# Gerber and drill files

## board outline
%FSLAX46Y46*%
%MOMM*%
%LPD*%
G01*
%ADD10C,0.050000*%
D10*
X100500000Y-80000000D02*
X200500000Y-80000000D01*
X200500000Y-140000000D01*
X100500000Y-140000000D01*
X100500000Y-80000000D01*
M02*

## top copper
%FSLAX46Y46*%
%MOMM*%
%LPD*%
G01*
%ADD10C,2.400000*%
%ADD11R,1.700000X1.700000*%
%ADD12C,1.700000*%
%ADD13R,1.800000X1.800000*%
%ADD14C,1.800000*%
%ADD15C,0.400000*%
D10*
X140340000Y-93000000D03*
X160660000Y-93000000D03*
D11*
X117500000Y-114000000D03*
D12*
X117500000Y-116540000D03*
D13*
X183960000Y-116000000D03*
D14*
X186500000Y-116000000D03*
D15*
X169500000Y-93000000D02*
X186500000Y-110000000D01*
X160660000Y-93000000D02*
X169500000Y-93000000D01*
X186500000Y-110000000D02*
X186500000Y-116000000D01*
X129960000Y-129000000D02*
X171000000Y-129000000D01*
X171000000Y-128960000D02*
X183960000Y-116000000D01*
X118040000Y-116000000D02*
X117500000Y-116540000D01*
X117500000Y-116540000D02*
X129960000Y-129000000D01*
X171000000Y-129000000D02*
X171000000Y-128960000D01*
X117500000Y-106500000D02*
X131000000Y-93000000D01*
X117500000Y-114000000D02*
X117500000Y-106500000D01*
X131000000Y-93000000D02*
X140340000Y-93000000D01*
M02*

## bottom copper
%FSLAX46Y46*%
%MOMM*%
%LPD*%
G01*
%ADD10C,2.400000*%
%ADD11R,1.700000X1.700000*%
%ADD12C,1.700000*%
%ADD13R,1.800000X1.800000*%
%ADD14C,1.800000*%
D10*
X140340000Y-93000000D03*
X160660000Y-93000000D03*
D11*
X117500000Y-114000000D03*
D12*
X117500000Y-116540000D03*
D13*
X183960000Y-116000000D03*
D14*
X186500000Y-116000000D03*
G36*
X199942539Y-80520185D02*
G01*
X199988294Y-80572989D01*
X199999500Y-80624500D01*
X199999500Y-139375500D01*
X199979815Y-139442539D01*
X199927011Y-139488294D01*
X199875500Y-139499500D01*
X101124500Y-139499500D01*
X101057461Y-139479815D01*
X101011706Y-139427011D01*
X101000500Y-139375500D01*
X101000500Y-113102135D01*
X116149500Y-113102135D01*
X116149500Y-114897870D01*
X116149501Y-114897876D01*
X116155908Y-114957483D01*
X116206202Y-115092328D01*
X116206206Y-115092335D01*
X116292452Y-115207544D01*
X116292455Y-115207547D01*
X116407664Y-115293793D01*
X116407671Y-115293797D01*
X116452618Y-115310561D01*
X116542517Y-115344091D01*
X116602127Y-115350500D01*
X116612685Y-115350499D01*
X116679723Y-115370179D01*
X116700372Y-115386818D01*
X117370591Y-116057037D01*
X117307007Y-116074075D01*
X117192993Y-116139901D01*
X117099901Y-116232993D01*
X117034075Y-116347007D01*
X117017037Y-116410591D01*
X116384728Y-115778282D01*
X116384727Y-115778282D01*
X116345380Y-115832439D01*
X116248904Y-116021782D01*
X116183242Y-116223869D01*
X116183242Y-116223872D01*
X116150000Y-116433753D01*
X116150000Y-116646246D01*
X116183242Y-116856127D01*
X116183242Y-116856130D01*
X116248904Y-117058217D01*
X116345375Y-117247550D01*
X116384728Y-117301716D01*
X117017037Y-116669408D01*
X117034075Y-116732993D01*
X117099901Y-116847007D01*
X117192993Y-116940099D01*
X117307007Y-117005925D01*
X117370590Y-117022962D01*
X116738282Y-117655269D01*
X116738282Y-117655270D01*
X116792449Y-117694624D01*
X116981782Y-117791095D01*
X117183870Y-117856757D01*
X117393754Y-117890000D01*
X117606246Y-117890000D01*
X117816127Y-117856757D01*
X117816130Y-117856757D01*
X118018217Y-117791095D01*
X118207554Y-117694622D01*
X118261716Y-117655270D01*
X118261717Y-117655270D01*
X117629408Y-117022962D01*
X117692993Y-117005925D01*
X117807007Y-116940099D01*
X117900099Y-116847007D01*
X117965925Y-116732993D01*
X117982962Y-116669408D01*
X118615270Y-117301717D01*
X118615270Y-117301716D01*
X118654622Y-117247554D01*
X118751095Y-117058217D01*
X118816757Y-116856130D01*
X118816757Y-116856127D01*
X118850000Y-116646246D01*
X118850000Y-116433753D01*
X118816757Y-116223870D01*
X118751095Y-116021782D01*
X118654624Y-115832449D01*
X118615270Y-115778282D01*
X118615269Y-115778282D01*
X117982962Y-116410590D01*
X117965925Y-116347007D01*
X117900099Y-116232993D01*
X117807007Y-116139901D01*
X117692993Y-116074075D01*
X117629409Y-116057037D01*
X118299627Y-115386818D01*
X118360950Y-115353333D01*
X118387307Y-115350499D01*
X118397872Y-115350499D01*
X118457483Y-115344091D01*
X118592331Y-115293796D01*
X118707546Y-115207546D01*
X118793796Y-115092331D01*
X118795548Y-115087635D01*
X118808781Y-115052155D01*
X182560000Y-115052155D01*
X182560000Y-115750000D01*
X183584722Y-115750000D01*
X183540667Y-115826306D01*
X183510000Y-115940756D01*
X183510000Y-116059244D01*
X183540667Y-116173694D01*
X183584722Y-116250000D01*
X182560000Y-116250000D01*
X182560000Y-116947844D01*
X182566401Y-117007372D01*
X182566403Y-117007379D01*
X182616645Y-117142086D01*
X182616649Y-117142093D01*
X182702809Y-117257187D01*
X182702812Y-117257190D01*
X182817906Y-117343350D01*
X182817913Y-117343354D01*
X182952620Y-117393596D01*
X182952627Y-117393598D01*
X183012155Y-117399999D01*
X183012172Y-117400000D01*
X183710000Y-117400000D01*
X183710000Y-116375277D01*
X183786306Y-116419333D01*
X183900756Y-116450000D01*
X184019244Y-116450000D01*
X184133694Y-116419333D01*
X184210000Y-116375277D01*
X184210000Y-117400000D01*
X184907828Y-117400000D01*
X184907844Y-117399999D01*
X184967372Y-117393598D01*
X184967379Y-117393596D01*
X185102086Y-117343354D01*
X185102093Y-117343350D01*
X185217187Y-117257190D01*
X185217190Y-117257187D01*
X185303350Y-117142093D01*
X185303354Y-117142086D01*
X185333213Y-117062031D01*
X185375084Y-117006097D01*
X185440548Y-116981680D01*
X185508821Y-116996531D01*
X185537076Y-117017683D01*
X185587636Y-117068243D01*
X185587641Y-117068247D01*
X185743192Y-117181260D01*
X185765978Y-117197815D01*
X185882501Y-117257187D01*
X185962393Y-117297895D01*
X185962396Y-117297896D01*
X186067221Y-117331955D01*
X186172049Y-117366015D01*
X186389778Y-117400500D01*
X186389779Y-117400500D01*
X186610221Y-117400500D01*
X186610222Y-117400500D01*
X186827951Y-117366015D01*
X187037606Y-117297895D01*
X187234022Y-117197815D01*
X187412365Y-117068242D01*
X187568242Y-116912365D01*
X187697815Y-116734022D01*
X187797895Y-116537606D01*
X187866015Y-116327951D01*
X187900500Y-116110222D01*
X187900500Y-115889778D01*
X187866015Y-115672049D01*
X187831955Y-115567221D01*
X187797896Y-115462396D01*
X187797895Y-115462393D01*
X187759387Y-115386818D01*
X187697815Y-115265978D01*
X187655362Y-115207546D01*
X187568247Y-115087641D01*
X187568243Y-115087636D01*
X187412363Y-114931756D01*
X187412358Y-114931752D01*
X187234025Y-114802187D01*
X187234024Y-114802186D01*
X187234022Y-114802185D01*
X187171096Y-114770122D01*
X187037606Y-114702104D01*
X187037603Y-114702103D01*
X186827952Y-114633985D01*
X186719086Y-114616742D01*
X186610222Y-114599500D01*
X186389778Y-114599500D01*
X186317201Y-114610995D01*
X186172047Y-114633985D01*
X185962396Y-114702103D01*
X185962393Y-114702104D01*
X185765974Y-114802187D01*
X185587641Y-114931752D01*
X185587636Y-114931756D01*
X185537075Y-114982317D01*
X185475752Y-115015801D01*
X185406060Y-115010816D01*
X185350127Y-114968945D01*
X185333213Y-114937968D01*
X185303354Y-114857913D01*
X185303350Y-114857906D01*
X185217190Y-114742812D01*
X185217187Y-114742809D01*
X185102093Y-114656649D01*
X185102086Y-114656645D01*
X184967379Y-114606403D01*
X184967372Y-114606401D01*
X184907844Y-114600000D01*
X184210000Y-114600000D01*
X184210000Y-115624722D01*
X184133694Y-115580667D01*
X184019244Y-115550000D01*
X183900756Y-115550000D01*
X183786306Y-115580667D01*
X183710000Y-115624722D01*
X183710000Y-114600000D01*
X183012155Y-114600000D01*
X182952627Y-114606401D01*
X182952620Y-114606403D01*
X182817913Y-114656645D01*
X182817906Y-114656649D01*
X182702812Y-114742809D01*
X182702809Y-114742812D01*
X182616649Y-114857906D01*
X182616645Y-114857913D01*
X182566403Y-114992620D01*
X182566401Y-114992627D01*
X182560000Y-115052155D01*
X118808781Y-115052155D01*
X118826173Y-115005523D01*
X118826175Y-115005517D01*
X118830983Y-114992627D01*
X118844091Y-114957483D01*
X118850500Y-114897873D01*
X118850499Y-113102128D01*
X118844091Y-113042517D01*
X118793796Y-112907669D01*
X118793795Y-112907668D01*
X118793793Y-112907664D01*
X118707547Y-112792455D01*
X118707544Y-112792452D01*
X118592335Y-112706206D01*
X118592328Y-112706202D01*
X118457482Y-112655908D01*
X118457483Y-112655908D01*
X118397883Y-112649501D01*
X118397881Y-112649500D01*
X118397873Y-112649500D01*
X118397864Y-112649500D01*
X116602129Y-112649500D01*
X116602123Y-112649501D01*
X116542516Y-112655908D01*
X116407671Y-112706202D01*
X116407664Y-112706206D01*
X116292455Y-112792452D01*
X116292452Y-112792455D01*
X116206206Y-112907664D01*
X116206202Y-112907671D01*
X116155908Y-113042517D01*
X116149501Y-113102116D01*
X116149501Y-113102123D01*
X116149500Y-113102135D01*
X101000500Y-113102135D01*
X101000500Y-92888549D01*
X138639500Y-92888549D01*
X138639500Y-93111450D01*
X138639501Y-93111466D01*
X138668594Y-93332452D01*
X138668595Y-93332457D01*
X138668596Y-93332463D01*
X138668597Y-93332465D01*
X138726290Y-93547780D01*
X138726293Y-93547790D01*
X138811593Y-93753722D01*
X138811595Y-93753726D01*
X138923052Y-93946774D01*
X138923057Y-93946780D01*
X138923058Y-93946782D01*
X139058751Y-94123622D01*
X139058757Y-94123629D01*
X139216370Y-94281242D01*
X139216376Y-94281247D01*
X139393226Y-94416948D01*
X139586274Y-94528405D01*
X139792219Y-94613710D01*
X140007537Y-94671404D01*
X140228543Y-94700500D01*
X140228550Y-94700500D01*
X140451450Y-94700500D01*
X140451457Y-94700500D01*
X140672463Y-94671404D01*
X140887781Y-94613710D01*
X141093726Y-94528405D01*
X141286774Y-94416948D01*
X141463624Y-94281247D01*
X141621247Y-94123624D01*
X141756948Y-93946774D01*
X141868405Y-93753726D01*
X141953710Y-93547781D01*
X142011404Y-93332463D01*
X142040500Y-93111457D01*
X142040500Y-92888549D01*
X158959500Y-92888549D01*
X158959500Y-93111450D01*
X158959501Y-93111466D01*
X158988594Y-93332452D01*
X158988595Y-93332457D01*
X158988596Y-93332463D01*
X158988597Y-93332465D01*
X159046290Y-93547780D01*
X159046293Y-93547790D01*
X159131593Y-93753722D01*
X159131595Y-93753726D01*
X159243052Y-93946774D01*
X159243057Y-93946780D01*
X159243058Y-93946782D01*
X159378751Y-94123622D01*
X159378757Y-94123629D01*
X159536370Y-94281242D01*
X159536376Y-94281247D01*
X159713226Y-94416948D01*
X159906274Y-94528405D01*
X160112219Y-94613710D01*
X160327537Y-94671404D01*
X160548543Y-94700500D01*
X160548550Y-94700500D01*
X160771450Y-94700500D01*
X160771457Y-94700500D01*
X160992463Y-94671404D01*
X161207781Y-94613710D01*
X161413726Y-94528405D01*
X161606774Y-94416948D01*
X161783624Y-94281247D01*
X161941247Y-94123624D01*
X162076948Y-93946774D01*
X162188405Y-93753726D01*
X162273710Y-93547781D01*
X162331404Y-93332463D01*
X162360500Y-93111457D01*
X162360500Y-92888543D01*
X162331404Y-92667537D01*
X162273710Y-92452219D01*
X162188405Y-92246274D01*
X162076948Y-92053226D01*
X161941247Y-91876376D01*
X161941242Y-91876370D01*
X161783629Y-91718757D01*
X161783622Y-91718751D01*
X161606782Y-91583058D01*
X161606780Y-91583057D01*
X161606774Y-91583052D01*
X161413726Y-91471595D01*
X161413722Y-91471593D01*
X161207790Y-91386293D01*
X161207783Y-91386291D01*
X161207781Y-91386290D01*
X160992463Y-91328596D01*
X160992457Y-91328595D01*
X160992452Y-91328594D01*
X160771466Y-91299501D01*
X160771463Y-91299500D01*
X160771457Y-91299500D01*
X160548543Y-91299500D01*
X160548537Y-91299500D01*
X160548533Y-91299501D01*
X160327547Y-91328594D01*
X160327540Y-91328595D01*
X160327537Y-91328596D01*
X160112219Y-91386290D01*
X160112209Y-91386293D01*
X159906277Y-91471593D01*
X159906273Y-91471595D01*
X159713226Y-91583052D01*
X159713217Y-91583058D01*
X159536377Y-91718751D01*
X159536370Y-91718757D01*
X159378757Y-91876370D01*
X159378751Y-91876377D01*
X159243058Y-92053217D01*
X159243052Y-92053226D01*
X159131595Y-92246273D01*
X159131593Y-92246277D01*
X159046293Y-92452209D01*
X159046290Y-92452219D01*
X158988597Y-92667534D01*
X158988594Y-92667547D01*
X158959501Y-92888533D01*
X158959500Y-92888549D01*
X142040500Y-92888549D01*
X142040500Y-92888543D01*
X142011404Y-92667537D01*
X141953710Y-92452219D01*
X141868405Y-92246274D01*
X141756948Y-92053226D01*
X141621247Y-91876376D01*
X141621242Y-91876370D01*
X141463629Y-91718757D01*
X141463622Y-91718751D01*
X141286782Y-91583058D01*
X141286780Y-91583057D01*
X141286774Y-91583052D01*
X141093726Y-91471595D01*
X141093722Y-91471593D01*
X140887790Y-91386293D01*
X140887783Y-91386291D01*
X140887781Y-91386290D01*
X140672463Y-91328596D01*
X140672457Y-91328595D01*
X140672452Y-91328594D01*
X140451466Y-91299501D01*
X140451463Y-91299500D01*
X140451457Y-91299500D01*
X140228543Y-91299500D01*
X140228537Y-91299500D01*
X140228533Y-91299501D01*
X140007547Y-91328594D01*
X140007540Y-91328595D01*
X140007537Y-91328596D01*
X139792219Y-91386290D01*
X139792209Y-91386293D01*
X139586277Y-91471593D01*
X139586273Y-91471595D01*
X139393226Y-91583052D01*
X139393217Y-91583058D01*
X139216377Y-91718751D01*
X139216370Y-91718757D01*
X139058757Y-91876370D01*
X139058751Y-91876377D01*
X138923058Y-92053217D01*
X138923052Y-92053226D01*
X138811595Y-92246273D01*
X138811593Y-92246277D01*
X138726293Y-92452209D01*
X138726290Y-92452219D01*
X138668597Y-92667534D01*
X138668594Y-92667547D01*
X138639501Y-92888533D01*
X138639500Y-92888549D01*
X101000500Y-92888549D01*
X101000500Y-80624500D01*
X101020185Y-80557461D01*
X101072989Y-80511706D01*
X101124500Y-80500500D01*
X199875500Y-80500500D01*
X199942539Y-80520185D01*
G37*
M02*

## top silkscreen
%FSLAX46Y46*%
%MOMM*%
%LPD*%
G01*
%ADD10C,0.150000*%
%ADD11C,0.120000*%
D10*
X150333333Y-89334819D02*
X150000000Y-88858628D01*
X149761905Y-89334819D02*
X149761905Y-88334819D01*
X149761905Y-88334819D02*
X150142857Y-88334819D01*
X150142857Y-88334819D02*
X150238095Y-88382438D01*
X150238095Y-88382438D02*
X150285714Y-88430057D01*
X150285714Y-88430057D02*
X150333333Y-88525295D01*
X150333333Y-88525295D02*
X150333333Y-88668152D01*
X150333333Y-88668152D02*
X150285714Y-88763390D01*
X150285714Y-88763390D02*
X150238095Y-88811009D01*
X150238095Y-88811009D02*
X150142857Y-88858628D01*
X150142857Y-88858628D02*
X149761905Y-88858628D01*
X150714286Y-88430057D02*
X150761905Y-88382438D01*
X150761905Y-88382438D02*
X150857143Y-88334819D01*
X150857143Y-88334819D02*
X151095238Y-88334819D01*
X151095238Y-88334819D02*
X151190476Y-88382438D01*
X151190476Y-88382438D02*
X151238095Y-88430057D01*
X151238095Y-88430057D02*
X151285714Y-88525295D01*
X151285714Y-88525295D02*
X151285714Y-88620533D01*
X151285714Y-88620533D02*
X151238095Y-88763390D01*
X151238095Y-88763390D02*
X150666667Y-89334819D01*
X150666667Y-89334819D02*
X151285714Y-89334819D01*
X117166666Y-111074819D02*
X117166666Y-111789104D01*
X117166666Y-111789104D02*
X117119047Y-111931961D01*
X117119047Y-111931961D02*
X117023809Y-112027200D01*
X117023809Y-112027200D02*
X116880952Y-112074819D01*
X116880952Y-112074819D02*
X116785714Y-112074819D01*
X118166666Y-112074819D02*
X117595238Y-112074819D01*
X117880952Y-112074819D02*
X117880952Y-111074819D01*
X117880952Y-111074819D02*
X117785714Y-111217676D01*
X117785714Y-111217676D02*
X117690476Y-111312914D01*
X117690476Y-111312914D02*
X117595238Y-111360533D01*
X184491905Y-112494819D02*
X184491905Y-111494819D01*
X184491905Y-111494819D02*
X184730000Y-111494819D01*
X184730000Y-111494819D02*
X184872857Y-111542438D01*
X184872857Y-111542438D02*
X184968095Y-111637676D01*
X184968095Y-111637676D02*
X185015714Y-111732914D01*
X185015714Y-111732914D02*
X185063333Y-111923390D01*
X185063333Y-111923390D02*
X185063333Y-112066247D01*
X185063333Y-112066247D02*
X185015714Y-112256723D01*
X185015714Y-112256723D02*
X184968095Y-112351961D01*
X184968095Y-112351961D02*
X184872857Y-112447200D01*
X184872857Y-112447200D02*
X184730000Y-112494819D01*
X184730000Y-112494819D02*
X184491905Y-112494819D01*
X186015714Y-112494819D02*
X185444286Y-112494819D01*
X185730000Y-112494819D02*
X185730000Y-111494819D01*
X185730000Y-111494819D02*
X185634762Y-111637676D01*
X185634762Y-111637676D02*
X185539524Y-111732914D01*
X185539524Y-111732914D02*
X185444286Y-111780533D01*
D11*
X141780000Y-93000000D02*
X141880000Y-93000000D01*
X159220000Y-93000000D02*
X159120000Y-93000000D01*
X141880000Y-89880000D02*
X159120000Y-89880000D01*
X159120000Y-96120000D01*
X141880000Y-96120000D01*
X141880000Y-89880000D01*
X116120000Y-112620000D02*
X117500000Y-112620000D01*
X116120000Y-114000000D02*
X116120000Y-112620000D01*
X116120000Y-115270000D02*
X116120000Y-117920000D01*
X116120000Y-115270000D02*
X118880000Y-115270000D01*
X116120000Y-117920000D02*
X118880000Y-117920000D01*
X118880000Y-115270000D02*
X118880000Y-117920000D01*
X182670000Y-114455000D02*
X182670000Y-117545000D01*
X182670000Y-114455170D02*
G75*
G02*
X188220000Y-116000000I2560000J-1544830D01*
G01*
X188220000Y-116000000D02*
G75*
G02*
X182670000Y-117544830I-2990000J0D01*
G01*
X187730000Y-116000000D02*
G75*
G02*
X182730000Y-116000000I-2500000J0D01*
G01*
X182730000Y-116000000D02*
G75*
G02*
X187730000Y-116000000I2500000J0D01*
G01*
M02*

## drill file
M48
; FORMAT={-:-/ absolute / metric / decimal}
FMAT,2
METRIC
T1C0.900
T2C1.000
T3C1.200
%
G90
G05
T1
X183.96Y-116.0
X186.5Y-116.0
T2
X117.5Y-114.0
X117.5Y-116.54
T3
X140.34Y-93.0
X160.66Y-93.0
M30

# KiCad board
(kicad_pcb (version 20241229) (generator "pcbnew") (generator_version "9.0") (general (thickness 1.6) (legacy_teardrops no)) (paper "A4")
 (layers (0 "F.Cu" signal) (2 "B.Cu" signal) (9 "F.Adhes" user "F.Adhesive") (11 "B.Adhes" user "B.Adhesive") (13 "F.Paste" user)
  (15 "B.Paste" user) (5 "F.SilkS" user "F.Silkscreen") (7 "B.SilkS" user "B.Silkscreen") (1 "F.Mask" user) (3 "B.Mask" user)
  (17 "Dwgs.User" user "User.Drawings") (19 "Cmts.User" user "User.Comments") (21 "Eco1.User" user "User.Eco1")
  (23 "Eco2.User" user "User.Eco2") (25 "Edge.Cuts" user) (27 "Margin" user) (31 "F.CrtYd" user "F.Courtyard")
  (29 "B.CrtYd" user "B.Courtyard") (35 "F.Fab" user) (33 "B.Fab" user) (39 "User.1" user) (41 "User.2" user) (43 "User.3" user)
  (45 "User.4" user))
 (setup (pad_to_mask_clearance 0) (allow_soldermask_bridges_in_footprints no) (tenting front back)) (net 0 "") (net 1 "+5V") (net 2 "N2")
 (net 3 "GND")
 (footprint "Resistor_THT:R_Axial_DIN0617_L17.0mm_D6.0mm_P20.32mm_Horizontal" (layer "F.Cu") (at 140.34 93)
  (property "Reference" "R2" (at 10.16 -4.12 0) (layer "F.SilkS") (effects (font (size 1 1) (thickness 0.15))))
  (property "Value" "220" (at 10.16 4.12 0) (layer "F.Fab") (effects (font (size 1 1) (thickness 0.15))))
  (fp_line (start 1.44 0) (end 1.54 0) (stroke (width 0.12) (type solid)) (layer "F.SilkS"))
  (fp_line (start 18.88 0) (end 18.78 0) (stroke (width 0.12) (type solid)) (layer "F.SilkS"))
  (fp_rect (start 1.54 -3.12) (end 18.78 3.12) (stroke (width 0.12) (type solid)) (fill no) (layer "F.SilkS"))
  (pad "1" thru_hole circle (at 0 0) (size 2.4 2.4) (drill 1.2) (layers "*.Cu" "*.Mask") (remove_unused_layers no) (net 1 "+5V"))
  (pad "2" thru_hole circle (at 20.32 0) (size 2.4 2.4) (drill 1.2) (layers "*.Cu" "*.Mask") (remove_unused_layers no) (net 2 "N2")))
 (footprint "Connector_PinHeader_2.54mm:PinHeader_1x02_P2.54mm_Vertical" (layer "F.Cu") (at 117.5 114)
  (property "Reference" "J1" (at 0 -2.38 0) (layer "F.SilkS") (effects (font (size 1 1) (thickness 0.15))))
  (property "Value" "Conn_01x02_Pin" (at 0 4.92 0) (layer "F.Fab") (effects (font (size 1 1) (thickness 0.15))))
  (fp_line (start -1.38 -1.38) (end 0 -1.38) (stroke (width 0.12) (type solid)) (layer "F.SilkS"))
  (fp_line (start -1.38 0) (end -1.38 -1.38) (stroke (width 0.12) (type solid)) (layer "F.SilkS"))
  (fp_line (start -1.38 1.27) (end -1.38 3.92) (stroke (width 0.12) (type solid)) (layer "F.SilkS"))
  (fp_line (start -1.38 1.27) (end 1.38 1.27) (stroke (width 0.12) (type solid)) (layer "F.SilkS"))
  (fp_line (start -1.38 3.92) (end 1.38 3.92) (stroke (width 0.12) (type solid)) (layer "F.SilkS"))
  (fp_line (start 1.38 1.27) (end 1.38 3.92) (stroke (width 0.12) (type solid)) (layer "F.SilkS"))
  (pad "1" thru_hole rect (at 0 0) (size 1.7 1.7) (drill 1) (layers "*.Cu" "*.Mask") (remove_unused_layers no) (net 1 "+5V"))
  (pad "2" thru_hole circle (at 0 2.54) (size 1.7 1.7) (drill 1) (layers "*.Cu" "*.Mask") (remove_unused_layers no) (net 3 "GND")))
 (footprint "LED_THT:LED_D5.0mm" (layer "F.Cu") (at 183.96 116)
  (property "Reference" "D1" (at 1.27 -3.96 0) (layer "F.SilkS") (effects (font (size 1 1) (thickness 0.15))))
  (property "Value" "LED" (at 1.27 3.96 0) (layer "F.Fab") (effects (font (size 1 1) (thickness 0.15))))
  (fp_line (start -1.29 -1.545) (end -1.29 1.545) (stroke (width 0.12) (type solid)) (layer "F.SilkS"))
  (fp_arc (start -1.29 -1.54483) (mid 2.071779 -2.880495) (end 4.26 0) (stroke (width 0.12) (type solid)) (layer "F.SilkS"))
  (fp_arc (start 4.26 0) (mid 2.071779 2.880495) (end -1.29 1.54483) (stroke (width 0.12) (type solid)) (layer "F.SilkS"))
  (fp_circle (center 1.27 0) (end 3.77 0) (stroke (width 0.12) (type solid)) (fill no) (layer "F.SilkS"))
  (pad "1" thru_hole rect (at 0 0) (size 1.8 1.8) (drill 0.9) (layers "*.Cu" "*.Mask") (remove_unused_layers no) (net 3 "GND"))
  (pad "2" thru_hole circle (at 2.54 0) (size 1.8 1.8) (drill 0.9) (layers "*.Cu" "*.Mask") (remove_unused_layers no) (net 2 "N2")))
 (gr_rect (start 100.5 80) (end 200.5 140) (stroke (width 0.05) (type default)) (fill no) (layer "Edge.Cuts"))
 (segment (start 169.5 93) (end 186.5 110) (width 0.4) (layer "F.Cu") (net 2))
 (segment (start 160.66 93) (end 169.5 93) (width 0.4) (layer "F.Cu") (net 2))
 (segment (start 186.5 110) (end 186.5 116) (width 0.4) (layer "F.Cu") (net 2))
 (segment (start 129.96 129) (end 171 129) (width 0.4) (layer "F.Cu") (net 3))
 (segment (start 171 128.96) (end 183.96 116) (width 0.4) (layer "F.Cu") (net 3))
 (segment (start 118.04 116) (end 117.5 116.54) (width 0.4) (layer "F.Cu") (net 3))
 (segment (start 117.5 116.54) (end 129.96 129) (width 0.4) (layer "F.Cu") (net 3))
 (segment (start 171 129) (end 171 128.96) (width 0.4) (layer "F.Cu") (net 3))
 (segment (start 117.5 106.5) (end 131 93) (width 0.4) (layer "F.Cu") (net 1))
 (segment (start 117.5 114) (end 117.5 106.5) (width 0.4) (layer "F.Cu") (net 1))
 (segment (start 131 93) (end 140.34 93) (width 0.4) (layer "F.Cu") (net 1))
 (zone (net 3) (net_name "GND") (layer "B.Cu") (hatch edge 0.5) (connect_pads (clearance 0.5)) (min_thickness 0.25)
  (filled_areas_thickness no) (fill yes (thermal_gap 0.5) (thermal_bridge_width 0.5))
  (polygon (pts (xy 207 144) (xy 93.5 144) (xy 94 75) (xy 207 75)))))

